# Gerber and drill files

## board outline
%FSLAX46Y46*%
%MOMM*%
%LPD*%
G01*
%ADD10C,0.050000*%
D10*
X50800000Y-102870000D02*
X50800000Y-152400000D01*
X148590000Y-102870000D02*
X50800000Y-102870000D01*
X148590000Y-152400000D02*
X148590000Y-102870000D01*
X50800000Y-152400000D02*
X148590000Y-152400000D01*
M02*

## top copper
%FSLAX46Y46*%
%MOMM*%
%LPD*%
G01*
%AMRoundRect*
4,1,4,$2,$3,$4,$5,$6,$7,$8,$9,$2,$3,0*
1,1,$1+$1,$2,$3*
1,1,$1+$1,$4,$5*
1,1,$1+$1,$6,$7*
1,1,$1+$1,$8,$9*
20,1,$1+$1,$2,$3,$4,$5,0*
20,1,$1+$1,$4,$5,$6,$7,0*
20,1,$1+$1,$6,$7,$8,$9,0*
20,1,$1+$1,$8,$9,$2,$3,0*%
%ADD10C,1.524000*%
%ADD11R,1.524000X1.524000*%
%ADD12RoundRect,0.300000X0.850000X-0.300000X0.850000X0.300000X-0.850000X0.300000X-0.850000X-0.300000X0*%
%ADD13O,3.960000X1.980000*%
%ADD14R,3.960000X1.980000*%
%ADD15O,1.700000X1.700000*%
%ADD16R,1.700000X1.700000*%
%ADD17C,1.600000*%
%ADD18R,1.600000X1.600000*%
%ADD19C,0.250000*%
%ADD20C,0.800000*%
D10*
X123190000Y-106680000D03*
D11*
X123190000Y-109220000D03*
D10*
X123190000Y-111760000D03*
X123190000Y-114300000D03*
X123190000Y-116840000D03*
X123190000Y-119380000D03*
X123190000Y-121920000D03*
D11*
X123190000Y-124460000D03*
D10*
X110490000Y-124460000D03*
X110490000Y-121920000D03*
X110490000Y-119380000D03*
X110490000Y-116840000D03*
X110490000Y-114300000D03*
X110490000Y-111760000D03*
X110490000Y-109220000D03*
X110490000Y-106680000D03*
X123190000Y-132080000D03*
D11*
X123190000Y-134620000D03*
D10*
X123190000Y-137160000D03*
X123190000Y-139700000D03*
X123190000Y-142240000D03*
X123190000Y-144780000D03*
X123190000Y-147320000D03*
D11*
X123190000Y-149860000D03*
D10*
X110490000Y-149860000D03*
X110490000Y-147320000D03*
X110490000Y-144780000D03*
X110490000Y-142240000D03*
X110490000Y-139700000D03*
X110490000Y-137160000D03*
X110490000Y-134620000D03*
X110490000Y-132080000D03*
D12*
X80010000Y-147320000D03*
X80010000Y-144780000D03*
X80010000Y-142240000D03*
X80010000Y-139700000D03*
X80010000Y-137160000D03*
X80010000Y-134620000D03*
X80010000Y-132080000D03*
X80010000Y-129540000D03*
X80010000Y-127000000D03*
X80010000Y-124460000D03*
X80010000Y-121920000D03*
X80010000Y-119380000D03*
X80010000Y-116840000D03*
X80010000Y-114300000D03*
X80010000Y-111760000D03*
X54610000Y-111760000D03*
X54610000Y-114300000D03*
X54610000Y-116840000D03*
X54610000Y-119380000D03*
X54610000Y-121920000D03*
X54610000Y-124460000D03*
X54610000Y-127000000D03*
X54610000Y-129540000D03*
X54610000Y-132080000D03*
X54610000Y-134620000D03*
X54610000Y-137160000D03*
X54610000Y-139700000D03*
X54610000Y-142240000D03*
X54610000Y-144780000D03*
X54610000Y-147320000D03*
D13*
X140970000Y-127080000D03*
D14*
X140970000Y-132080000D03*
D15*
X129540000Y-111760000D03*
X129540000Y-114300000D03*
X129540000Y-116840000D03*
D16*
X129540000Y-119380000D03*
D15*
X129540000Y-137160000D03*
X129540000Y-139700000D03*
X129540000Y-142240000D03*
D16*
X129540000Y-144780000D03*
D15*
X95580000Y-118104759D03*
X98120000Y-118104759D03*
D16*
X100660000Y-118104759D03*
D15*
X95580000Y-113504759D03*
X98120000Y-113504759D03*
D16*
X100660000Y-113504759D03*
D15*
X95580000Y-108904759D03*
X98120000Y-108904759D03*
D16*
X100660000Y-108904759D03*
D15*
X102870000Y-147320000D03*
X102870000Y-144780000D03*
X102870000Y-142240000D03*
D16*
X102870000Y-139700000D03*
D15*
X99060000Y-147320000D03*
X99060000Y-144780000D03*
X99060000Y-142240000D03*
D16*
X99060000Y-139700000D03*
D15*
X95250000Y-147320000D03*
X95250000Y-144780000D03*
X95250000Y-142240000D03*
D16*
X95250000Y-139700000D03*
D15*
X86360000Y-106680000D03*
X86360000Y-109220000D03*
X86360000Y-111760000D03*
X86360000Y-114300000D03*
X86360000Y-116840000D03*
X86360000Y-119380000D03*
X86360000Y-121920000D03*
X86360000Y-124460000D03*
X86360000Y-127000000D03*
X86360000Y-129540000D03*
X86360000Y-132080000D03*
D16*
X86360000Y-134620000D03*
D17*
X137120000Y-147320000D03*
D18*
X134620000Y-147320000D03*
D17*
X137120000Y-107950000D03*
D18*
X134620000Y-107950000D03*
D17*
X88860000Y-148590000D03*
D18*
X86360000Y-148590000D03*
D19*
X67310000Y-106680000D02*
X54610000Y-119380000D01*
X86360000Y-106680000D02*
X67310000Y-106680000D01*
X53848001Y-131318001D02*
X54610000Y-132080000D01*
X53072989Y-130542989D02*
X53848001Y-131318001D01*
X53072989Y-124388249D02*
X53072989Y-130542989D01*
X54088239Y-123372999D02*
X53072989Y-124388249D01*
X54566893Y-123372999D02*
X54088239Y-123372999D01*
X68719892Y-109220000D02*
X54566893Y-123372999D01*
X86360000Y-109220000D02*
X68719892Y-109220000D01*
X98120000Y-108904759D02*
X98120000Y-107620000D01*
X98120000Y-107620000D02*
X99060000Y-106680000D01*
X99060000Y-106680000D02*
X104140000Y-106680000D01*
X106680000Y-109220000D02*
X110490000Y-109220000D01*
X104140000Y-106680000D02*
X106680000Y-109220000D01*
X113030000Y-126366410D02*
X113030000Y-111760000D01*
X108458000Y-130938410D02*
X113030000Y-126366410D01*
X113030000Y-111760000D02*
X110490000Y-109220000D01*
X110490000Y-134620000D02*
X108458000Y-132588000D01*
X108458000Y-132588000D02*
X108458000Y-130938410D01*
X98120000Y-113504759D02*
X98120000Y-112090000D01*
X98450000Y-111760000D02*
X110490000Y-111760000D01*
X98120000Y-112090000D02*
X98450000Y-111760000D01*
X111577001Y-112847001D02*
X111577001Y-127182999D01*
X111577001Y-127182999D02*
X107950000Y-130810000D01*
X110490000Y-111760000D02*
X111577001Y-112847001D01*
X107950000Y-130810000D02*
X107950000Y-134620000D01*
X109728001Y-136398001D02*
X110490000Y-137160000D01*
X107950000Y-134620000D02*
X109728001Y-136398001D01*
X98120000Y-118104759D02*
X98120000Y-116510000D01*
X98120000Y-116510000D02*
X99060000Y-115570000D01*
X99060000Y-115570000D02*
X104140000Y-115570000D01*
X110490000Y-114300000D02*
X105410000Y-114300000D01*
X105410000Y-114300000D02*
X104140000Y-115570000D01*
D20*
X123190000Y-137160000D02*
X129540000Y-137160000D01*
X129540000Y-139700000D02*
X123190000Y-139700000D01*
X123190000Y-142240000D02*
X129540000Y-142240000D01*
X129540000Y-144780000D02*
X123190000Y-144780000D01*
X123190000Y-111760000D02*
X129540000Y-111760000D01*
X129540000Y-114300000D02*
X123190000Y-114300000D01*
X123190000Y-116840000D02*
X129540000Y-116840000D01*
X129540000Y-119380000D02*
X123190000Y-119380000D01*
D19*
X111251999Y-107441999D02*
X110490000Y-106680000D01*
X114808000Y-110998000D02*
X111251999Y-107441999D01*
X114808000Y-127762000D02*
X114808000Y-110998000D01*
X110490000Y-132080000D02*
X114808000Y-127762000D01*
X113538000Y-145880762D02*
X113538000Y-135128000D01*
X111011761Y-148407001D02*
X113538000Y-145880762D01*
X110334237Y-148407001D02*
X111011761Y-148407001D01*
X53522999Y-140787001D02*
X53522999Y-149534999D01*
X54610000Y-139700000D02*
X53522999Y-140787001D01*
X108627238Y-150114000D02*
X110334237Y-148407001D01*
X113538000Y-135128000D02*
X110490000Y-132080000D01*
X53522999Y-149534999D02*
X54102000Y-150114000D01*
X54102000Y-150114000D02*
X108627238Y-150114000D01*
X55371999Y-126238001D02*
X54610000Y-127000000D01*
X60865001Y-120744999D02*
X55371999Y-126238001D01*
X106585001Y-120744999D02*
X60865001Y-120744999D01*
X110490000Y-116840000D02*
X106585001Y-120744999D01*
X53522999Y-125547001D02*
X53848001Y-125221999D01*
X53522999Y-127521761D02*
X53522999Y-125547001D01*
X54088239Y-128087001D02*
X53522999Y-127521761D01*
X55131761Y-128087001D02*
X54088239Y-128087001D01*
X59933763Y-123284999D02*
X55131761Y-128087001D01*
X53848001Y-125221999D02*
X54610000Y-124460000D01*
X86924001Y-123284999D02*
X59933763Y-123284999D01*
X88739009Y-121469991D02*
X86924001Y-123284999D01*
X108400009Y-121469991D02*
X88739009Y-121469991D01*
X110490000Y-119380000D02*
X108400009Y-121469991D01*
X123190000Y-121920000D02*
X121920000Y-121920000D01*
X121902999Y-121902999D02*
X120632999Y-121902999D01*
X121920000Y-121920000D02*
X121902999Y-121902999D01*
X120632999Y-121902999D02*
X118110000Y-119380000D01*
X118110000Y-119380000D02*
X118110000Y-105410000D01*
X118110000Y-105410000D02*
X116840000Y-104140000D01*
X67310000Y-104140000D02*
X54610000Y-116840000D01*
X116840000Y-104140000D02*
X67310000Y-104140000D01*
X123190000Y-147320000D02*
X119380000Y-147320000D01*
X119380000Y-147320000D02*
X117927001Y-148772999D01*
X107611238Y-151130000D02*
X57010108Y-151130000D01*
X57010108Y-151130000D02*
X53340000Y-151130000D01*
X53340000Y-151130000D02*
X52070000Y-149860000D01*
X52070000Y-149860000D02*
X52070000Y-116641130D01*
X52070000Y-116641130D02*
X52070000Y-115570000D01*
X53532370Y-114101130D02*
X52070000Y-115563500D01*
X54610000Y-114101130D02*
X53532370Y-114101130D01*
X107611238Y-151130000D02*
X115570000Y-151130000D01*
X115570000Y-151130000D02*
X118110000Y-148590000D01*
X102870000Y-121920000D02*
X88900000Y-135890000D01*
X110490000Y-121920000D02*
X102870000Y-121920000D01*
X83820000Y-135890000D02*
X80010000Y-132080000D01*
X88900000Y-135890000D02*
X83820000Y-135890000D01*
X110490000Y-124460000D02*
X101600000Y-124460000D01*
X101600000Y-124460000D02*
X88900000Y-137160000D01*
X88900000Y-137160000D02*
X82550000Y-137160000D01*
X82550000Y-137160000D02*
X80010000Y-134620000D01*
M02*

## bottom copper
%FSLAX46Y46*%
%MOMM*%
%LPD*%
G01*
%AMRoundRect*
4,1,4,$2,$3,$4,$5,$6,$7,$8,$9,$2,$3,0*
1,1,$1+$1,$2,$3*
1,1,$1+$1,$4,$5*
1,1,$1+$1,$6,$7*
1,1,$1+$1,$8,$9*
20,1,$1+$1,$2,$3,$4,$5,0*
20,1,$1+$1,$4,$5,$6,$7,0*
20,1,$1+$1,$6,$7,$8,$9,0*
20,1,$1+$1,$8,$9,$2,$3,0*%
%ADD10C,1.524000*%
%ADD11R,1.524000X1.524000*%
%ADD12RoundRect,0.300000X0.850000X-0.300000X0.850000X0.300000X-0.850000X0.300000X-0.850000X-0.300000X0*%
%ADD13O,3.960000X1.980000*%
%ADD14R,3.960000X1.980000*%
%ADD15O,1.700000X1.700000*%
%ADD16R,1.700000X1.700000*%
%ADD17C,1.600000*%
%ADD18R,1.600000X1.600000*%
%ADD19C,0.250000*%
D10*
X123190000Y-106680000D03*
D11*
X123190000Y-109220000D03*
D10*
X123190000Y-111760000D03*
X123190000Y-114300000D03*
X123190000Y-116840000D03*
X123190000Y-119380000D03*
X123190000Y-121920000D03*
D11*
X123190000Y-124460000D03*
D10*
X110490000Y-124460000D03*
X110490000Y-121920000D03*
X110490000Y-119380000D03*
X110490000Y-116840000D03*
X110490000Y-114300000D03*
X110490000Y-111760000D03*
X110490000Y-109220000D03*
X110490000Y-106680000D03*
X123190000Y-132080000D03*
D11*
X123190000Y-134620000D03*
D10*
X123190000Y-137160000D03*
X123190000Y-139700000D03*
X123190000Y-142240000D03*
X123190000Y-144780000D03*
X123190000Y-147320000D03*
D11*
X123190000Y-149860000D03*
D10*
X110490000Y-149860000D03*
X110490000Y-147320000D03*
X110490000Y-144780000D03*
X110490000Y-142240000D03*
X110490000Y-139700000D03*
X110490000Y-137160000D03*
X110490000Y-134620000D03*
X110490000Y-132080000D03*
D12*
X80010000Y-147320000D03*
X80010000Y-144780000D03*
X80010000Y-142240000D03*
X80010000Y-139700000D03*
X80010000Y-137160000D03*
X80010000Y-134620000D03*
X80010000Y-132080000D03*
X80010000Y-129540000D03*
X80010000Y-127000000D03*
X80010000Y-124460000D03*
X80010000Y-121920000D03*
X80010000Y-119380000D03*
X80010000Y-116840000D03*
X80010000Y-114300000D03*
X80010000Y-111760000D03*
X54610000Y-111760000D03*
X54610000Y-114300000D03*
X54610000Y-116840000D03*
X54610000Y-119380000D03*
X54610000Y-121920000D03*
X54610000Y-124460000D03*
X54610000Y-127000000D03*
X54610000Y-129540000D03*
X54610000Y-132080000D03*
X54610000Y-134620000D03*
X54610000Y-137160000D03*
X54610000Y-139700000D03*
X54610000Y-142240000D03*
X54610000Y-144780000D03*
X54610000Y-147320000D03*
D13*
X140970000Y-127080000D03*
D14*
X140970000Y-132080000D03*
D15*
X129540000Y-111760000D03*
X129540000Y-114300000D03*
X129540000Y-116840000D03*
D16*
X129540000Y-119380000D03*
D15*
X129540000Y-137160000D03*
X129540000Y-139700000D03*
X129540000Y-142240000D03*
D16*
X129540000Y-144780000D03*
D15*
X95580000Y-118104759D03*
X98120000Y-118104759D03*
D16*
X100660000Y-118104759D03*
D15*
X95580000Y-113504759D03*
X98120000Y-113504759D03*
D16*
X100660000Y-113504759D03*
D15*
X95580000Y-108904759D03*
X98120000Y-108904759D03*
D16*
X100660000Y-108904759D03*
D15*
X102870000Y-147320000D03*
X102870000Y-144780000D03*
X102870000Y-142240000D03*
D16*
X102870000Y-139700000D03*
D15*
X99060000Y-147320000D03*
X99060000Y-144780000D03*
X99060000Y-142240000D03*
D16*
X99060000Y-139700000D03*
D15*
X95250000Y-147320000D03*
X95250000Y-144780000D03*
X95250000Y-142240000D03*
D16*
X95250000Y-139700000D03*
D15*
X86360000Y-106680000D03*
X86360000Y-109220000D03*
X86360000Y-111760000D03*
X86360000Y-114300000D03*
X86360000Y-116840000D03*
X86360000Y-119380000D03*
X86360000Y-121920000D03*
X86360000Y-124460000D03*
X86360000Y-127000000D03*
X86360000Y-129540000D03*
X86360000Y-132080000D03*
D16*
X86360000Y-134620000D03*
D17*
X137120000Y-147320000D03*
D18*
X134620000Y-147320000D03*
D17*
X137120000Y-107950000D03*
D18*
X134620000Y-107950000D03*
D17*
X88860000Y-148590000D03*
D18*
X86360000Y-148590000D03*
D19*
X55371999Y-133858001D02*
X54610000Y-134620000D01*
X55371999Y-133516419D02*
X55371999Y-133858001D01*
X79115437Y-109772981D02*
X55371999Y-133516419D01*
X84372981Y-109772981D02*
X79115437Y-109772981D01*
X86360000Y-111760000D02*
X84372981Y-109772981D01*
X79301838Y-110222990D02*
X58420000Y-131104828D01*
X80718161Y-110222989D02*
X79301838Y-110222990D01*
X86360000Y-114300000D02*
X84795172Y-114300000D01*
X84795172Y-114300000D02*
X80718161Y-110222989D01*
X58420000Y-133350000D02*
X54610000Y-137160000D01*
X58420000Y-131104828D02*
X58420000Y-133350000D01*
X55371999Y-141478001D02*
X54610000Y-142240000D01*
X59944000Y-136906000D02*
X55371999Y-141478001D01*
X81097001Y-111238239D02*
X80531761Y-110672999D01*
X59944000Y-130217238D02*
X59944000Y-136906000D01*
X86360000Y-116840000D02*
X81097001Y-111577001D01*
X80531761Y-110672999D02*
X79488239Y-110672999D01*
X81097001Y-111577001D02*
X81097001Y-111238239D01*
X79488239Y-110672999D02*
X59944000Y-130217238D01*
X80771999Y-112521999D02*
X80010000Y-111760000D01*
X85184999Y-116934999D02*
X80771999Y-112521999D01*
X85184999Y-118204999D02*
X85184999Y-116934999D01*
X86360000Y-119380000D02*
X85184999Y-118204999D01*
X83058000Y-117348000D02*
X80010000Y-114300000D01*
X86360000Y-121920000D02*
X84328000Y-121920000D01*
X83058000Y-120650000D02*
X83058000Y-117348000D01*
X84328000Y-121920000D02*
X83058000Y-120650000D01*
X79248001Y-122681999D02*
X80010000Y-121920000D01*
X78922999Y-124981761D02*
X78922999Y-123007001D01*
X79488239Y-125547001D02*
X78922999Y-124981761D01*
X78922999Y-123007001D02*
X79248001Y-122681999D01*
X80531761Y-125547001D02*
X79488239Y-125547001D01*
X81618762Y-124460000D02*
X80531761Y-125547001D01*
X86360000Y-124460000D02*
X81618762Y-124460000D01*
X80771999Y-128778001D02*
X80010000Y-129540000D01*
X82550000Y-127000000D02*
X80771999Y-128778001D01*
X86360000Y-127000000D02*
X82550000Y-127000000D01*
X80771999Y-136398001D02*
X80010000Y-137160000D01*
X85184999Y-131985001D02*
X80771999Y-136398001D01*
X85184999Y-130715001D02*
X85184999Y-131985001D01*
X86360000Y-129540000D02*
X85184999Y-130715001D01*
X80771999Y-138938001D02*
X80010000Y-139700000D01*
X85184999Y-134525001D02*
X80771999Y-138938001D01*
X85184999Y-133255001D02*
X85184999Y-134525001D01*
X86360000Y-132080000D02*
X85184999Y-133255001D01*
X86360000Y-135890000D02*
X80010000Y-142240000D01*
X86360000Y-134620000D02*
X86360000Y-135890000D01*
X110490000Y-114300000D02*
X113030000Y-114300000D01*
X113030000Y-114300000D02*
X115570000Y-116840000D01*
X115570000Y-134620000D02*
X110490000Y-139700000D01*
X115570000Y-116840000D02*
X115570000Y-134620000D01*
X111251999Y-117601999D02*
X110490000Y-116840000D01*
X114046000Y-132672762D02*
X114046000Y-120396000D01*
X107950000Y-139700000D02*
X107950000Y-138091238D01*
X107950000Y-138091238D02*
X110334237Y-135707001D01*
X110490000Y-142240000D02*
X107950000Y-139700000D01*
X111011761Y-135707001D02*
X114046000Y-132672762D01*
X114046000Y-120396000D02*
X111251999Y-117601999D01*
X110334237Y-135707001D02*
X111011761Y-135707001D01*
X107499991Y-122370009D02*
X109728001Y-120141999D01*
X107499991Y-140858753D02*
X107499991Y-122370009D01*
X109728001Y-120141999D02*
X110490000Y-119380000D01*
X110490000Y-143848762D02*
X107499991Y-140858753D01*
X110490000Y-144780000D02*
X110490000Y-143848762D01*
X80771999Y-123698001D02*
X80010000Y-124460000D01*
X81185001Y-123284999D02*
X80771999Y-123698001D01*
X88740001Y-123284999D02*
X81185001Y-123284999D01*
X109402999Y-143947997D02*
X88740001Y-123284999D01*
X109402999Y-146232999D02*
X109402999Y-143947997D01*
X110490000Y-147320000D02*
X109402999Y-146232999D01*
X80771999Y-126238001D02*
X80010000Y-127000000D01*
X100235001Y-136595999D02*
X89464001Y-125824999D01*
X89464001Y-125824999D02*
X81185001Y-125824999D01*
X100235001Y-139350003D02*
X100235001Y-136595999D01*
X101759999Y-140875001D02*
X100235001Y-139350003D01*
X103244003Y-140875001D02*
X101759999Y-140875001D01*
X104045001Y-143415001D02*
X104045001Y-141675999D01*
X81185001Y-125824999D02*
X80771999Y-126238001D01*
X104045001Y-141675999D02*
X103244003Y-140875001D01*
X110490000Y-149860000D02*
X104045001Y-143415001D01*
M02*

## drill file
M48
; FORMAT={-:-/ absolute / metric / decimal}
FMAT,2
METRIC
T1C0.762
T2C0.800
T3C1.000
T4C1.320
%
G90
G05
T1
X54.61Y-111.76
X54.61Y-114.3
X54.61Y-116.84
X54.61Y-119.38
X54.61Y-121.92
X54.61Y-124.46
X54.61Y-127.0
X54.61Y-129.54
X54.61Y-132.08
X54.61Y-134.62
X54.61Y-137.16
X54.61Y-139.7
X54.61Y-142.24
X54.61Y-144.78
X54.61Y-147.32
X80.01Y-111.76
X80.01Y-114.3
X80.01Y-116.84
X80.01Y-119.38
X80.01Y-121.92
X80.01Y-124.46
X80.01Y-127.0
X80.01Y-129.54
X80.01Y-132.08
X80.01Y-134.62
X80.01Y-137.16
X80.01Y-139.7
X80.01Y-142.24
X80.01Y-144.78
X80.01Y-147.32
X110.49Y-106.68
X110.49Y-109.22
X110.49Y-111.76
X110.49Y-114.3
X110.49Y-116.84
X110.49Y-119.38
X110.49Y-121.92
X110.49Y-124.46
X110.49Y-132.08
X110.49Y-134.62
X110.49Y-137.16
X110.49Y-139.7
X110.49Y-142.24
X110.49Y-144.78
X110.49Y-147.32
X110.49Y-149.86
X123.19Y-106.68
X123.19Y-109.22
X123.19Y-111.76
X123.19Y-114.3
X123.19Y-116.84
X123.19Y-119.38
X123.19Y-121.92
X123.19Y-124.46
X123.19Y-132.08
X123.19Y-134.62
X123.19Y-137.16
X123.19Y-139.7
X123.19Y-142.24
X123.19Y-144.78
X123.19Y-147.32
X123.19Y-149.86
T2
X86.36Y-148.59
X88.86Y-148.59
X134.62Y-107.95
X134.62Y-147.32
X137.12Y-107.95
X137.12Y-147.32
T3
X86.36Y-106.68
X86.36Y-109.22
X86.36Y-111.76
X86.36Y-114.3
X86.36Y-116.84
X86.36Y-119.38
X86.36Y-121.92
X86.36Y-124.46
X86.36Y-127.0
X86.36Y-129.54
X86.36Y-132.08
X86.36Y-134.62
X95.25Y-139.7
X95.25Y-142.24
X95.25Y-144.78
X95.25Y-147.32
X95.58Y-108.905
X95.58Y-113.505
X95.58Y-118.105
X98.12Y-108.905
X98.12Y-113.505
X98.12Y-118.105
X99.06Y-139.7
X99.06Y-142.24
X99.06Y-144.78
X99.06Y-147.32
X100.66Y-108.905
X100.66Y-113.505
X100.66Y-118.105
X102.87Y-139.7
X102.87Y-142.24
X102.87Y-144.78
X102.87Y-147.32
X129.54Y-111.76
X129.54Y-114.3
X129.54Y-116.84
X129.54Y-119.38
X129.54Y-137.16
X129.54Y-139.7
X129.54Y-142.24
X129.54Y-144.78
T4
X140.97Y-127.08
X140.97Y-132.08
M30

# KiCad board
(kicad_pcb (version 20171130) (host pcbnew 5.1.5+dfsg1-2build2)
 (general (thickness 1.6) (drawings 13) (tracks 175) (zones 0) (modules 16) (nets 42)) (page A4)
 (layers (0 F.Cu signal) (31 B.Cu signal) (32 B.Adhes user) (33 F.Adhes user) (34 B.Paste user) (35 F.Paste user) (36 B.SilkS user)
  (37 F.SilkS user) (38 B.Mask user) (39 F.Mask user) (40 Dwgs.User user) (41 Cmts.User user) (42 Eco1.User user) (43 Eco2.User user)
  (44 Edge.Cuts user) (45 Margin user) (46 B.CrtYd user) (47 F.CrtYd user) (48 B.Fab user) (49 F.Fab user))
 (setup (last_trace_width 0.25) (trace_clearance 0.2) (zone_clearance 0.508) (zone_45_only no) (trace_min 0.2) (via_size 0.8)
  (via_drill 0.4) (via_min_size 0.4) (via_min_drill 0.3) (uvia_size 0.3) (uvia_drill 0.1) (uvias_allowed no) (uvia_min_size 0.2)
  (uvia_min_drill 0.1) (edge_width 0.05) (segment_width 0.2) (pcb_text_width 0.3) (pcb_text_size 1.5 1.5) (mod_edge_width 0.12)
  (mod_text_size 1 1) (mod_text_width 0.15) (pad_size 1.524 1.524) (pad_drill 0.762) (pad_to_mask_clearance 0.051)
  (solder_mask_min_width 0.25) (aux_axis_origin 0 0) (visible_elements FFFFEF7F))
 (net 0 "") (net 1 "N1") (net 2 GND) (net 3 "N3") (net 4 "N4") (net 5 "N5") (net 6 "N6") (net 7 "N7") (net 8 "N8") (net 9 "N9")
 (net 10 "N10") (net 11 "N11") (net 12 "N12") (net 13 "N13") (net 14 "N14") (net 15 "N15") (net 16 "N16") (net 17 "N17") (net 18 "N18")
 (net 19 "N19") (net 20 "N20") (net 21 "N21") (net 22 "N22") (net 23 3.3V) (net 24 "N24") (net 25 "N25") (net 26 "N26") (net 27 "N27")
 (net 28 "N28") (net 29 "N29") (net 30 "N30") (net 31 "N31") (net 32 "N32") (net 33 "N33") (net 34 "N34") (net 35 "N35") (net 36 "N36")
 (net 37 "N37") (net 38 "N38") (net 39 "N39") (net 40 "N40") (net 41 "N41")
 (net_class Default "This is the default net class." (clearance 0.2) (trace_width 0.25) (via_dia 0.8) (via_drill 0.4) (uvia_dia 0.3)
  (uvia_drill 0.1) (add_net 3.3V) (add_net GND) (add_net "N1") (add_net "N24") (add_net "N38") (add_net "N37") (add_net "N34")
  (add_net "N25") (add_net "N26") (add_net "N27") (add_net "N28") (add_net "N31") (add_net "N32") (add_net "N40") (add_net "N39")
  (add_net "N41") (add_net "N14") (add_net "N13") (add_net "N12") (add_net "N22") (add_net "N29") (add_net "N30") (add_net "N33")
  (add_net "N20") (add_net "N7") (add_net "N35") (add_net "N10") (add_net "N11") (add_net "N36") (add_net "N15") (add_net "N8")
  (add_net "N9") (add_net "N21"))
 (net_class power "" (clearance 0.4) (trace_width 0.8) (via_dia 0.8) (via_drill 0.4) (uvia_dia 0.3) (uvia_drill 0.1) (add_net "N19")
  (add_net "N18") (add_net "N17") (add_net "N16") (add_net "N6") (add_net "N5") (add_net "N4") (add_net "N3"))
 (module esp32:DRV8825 (layer F.Cu) (at 116.84 115.57)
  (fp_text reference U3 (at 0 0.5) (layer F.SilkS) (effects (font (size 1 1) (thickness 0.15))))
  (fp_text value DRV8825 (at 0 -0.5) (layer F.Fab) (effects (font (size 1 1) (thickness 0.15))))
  (pad 16 thru_hole circle (at 6.35 -8.89) (size 1.524 1.524) (drill 0.762) (layers *.Cu *.Mask) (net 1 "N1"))
  (pad 15 thru_hole rect (at 6.35 -6.35) (size 1.524 1.524) (drill 0.762) (layers *.Cu *.Mask) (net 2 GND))
  (pad 14 thru_hole circle (at 6.35 -3.81) (size 1.524 1.524) (drill 0.762) (layers *.Cu *.Mask) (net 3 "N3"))
  (pad 13 thru_hole circle (at 6.35 -1.27) (size 1.524 1.524) (drill 0.762) (layers *.Cu *.Mask) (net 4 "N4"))
  (pad 12 thru_hole circle (at 6.35 1.27) (size 1.524 1.524) (drill 0.762) (layers *.Cu *.Mask) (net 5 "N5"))
  (pad 11 thru_hole circle (at 6.35 3.81) (size 1.524 1.524) (drill 0.762) (layers *.Cu *.Mask) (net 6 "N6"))
  (pad 10 thru_hole circle (at 6.35 6.35) (size 1.524 1.524) (drill 0.762) (layers *.Cu *.Mask) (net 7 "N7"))
  (pad 9 thru_hole rect (at 6.35 8.89) (size 1.524 1.524) (drill 0.762) (layers *.Cu *.Mask) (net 2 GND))
  (pad 8 thru_hole circle (at -6.35 8.89) (size 1.524 1.524) (drill 0.762) (layers *.Cu *.Mask) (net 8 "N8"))
  (pad 7 thru_hole circle (at -6.35 6.35) (size 1.524 1.524) (drill 0.762) (layers *.Cu *.Mask) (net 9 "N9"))
  (pad 6 thru_hole circle (at -6.35 3.81) (size 1.524 1.524) (drill 0.762) (layers *.Cu *.Mask) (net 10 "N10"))
  (pad 5 thru_hole circle (at -6.35 1.27) (size 1.524 1.524) (drill 0.762) (layers *.Cu *.Mask) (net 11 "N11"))
  (pad 4 thru_hole circle (at -6.35 -1.27) (size 1.524 1.524) (drill 0.762) (layers *.Cu *.Mask) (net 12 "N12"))
  (pad 3 thru_hole circle (at -6.35 -3.81) (size 1.524 1.524) (drill 0.762) (layers *.Cu *.Mask) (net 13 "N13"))
  (pad 2 thru_hole circle (at -6.35 -6.35) (size 1.524 1.524) (drill 0.762) (layers *.Cu *.Mask) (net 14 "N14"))
  (pad 1 thru_hole circle (at -6.35 -8.89) (size 1.524 1.524) (drill 0.762) (layers *.Cu *.Mask) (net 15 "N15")))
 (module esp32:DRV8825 (layer F.Cu) (at 116.84 140.97)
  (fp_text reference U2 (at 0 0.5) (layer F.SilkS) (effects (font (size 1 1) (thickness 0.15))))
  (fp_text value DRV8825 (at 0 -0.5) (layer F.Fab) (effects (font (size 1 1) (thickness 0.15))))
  (pad 16 thru_hole circle (at 6.35 -8.89) (size 1.524 1.524) (drill 0.762) (layers *.Cu *.Mask) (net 1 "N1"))
  (pad 15 thru_hole rect (at 6.35 -6.35) (size 1.524 1.524) (drill 0.762) (layers *.Cu *.Mask) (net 2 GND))
  (pad 14 thru_hole circle (at 6.35 -3.81) (size 1.524 1.524) (drill 0.762) (layers *.Cu *.Mask) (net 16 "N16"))
  (pad 13 thru_hole circle (at 6.35 -1.27) (size 1.524 1.524) (drill 0.762) (layers *.Cu *.Mask) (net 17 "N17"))
  (pad 12 thru_hole circle (at 6.35 1.27) (size 1.524 1.524) (drill 0.762) (layers *.Cu *.Mask) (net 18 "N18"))
  (pad 11 thru_hole circle (at 6.35 3.81) (size 1.524 1.524) (drill 0.762) (layers *.Cu *.Mask) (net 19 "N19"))
  (pad 10 thru_hole circle (at 6.35 6.35) (size 1.524 1.524) (drill 0.762) (layers *.Cu *.Mask) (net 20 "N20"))
  (pad 9 thru_hole rect (at 6.35 8.89) (size 1.524 1.524) (drill 0.762) (layers *.Cu *.Mask) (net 2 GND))
  (pad 8 thru_hole circle (at -6.35 8.89) (size 1.524 1.524) (drill 0.762) (layers *.Cu *.Mask) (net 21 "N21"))
  (pad 7 thru_hole circle (at -6.35 6.35) (size 1.524 1.524) (drill 0.762) (layers *.Cu *.Mask) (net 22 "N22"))
  (pad 6 thru_hole circle (at -6.35 3.81) (size 1.524 1.524) (drill 0.762) (layers *.Cu *.Mask) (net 10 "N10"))
  (pad 5 thru_hole circle (at -6.35 1.27) (size 1.524 1.524) (drill 0.762) (layers *.Cu *.Mask) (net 11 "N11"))
  (pad 4 thru_hole circle (at -6.35 -1.27) (size 1.524 1.524) (drill 0.762) (layers *.Cu *.Mask) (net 12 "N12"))
  (pad 3 thru_hole circle (at -6.35 -3.81) (size 1.524 1.524) (drill 0.762) (layers *.Cu *.Mask) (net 13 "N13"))
  (pad 2 thru_hole circle (at -6.35 -6.35) (size 1.524 1.524) (drill 0.762) (layers *.Cu *.Mask) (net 14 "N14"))
  (pad 1 thru_hole circle (at -6.35 -8.89) (size 1.524 1.524) (drill 0.762) (layers *.Cu *.Mask) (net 15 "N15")))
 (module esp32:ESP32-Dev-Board (layer F.Cu) (at 67.31 129.54 90)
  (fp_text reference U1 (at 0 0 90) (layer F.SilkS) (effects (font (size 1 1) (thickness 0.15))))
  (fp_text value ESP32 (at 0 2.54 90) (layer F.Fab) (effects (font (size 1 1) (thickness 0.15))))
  (pad 1 thru_hole roundrect (at -17.78 12.7 90) (size 1.2 2.3) (drill 0.762) (layers *.Cu *.Mask) (roundrect_rratio 0.25) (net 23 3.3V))
  (pad 2 thru_hole roundrect (at -15.24 12.7 90) (size 1.2 2.3) (drill 0.762) (layers *.Cu *.Mask) (roundrect_rratio 0.25) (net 2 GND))
  (pad 3 thru_hole roundrect (at -12.7 12.7 90) (size 1.2 2.3) (drill 0.762) (layers *.Cu *.Mask) (roundrect_rratio 0.25) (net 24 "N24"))
  (pad 4 thru_hole roundrect (at -10.16 12.7 90) (size 1.2 2.3) (drill 0.762) (layers *.Cu *.Mask) (roundrect_rratio 0.25) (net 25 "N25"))
  (pad 5 thru_hole roundrect (at -7.62 12.7 90) (size 1.2 2.3) (drill 0.762) (layers *.Cu *.Mask) (roundrect_rratio 0.25) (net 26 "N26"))
  (pad 6 thru_hole roundrect (at -5.08 12.7 90) (size 1.2 2.3) (drill 0.762) (layers *.Cu *.Mask) (roundrect_rratio 0.25) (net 8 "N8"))
  (pad 7 thru_hole roundrect (at -2.54 12.7 90) (size 1.2 2.3) (drill 0.762) (layers *.Cu *.Mask) (roundrect_rratio 0.25) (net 9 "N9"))
  (pad 8 thru_hole roundrect (at 0 12.7 90) (size 1.2 2.3) (drill 0.762) (layers *.Cu *.Mask) (roundrect_rratio 0.25) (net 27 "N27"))
  (pad 9 thru_hole roundrect (at 2.54 12.7 90) (size 1.2 2.3) (drill 0.762) (layers *.Cu *.Mask) (roundrect_rratio 0.25) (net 21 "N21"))
  (pad 10 thru_hole roundrect (at 5.08 12.7 90) (size 1.2 2.3) (drill 0.762) (layers *.Cu *.Mask) (roundrect_rratio 0.25) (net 22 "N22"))
  (pad 11 thru_hole roundrect (at 7.62 12.7 90) (size 1.2 2.3) (drill 0.762) (layers *.Cu *.Mask) (roundrect_rratio 0.25) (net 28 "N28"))
  (pad 12 thru_hole roundrect (at 10.16 12.7 90) (size 1.2 2.3) (drill 0.762) (layers *.Cu *.Mask) (roundrect_rratio 0.25) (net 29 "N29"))
  (pad 13 thru_hole roundrect (at 12.7 12.7 90) (size 1.2 2.3) (drill 0.762) (layers *.Cu *.Mask) (roundrect_rratio 0.25) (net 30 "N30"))
  (pad 14 thru_hole roundrect (at 15.24 12.7 90) (size 1.2 2.3) (drill 0.762) (layers *.Cu *.Mask) (roundrect_rratio 0.25) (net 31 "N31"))
  (pad 15 thru_hole roundrect (at 17.78 12.7 90) (size 1.2 2.3) (drill 0.762) (layers *.Cu *.Mask) (roundrect_rratio 0.25) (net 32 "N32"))
  (pad 16 thru_hole roundrect (at 17.78 -12.7 90) (size 1.2 2.3) (drill 0.762) (layers *.Cu *.Mask) (roundrect_rratio 0.25) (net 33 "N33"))
  (pad 17 thru_hole roundrect (at 15.24 -12.7 90) (size 1.2 2.3) (drill 0.762) (layers *.Cu *.Mask) (roundrect_rratio 0.25) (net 20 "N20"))
  (pad 18 thru_hole roundrect (at 12.7 -12.7 90) (size 1.2 2.3) (drill 0.762) (layers *.Cu *.Mask) (roundrect_rratio 0.25) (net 7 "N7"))
  (pad 19 thru_hole roundrect (at 10.16 -12.7 90) (size 1.2 2.3) (drill 0.762) (layers *.Cu *.Mask) (roundrect_rratio 0.25) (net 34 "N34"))
  (pad 20 thru_hole roundrect (at 7.62 -12.7 90) (size 1.2 2.3) (drill 0.762) (layers *.Cu *.Mask) (roundrect_rratio 0.25) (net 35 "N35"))
  (pad 21 thru_hole roundrect (at 5.08 -12.7 90) (size 1.2 2.3) (drill 0.762) (layers *.Cu *.Mask) (roundrect_rratio 0.25) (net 10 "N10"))
  (pad 22 thru_hole roundrect (at 2.54 -12.7 90) (size 1.2 2.3) (drill 0.762) (layers *.Cu *.Mask) (roundrect_rratio 0.25) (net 11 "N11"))
  (pad 23 thru_hole roundrect (at 0 -12.7 90) (size 1.2 2.3) (drill 0.762) (layers *.Cu *.Mask) (roundrect_rratio 0.25) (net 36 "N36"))
  (pad 24 thru_hole roundrect (at -2.54 -12.7 90) (size 1.2 2.3) (drill 0.762) (layers *.Cu *.Mask) (roundrect_rratio 0.25) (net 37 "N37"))
  (pad 25 thru_hole roundrect (at -5.08 -12.7 90) (size 1.2 2.3) (drill 0.762) (layers *.Cu *.Mask) (roundrect_rratio 0.25) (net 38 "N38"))
  (pad 26 thru_hole roundrect (at -7.62 -12.7 90) (size 1.2 2.3) (drill 0.762) (layers *.Cu *.Mask) (roundrect_rratio 0.25) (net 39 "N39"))
  (pad 27 thru_hole roundrect (at -10.16 -12.7 90) (size 1.2 2.3) (drill 0.762) (layers *.Cu *.Mask) (roundrect_rratio 0.25) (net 15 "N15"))
  (pad 28 thru_hole roundrect (at -12.7 -12.7 90) (size 1.2 2.3) (drill 0.762) (layers *.Cu *.Mask) (roundrect_rratio 0.25) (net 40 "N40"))
  (pad 29 thru_hole roundrect (at -15.24 -12.7 90) (size 1.2 2.3) (drill 0.762) (layers *.Cu *.Mask) (roundrect_rratio 0.25) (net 2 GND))
  (pad 30 thru_hole roundrect (at -17.78 -12.7 90) (size 1.2 2.3) (drill 0.762) (layers *.Cu *.Mask) (roundrect_rratio 0.25) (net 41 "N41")))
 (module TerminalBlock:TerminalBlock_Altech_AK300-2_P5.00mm (layer F.Cu) (at 140.97 132.08 90)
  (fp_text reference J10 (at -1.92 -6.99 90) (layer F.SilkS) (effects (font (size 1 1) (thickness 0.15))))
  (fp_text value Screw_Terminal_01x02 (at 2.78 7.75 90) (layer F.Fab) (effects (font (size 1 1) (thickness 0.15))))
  (pad 2 thru_hole oval (at 5 0 90) (size 1.98 3.96) (drill 1.32) (layers *.Cu *.Mask) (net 1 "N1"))
  (pad 1 thru_hole rect (at 0 0 90) (size 1.98 3.96) (drill 1.32) (layers *.Cu *.Mask) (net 2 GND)))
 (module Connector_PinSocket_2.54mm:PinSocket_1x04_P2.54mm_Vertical (layer F.Cu) (at 129.54 119.38 180)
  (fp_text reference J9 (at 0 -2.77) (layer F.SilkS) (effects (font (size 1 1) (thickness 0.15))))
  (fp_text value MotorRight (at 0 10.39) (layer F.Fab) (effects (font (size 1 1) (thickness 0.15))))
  (pad 4 thru_hole oval (at 0 7.62 180) (size 1.7 1.7) (drill 1) (layers *.Cu *.Mask) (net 3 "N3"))
  (pad 3 thru_hole oval (at 0 5.08 180) (size 1.7 1.7) (drill 1) (layers *.Cu *.Mask) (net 4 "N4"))
  (pad 2 thru_hole oval (at 0 2.54 180) (size 1.7 1.7) (drill 1) (layers *.Cu *.Mask) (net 5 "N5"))
  (pad 1 thru_hole rect (at 0 0 180) (size 1.7 1.7) (drill 1) (layers *.Cu *.Mask) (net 6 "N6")))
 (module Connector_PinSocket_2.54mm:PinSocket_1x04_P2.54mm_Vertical (layer F.Cu) (at 129.54 144.78 180)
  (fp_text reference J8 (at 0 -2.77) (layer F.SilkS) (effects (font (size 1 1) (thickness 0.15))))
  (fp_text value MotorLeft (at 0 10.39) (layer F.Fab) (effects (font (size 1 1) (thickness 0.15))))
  (pad 4 thru_hole oval (at 0 7.62 180) (size 1.7 1.7) (drill 1) (layers *.Cu *.Mask) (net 16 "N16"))
  (pad 3 thru_hole oval (at 0 5.08 180) (size 1.7 1.7) (drill 1) (layers *.Cu *.Mask) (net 17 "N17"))
  (pad 2 thru_hole oval (at 0 2.54 180) (size 1.7 1.7) (drill 1) (layers *.Cu *.Mask) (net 18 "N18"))
  (pad 1 thru_hole rect (at 0 0 180) (size 1.7 1.7) (drill 1) (layers *.Cu *.Mask) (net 19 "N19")))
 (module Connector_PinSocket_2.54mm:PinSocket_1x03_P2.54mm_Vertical (layer F.Cu) (at 100.66 118.104759 270)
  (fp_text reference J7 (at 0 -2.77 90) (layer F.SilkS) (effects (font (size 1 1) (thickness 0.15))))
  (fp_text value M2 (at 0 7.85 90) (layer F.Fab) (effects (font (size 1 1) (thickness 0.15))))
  (pad 3 thru_hole oval (at 0 5.08 270) (size 1.7 1.7) (drill 1) (layers *.Cu *.Mask) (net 23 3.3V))
  (pad 2 thru_hole oval (at 0 2.54 270) (size 1.7 1.7) (drill 1) (layers *.Cu *.Mask) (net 12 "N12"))
  (pad 1 thru_hole rect (at 0 0 270) (size 1.7 1.7) (drill 1) (layers *.Cu *.Mask) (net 2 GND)))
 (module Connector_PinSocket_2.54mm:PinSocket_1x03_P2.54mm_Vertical (layer F.Cu) (at 100.66 113.504759 270)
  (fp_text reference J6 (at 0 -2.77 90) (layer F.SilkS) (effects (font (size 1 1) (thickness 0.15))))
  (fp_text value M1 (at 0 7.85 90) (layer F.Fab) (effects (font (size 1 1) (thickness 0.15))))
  (pad 3 thru_hole oval (at 0 5.08 270) (size 1.7 1.7) (drill 1) (layers *.Cu *.Mask) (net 23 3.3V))
  (pad 2 thru_hole oval (at 0 2.54 270) (size 1.7 1.7) (drill 1) (layers *.Cu *.Mask) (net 13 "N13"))
  (pad 1 thru_hole rect (at 0 0 270) (size 1.7 1.7) (drill 1) (layers *.Cu *.Mask) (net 2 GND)))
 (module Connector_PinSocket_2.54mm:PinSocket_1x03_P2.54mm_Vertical (layer F.Cu) (at 100.66 108.904759 270)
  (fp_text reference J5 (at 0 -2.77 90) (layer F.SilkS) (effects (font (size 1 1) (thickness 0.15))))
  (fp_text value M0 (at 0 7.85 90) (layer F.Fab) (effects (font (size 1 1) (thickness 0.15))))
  (pad 3 thru_hole oval (at 0 5.08 270) (size 1.7 1.7) (drill 1) (layers *.Cu *.Mask) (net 23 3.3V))
  (pad 2 thru_hole oval (at 0 2.54 270) (size 1.7 1.7) (drill 1) (layers *.Cu *.Mask) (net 14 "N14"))
  (pad 1 thru_hole rect (at 0 0 270) (size 1.7 1.7) (drill 1) (layers *.Cu *.Mask) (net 2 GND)))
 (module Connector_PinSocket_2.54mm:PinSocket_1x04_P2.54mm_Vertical (layer F.Cu) (at 102.87 139.7)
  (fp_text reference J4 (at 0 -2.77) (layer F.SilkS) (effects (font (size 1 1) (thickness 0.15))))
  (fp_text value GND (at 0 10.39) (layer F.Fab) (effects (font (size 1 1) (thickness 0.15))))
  (pad 4 thru_hole oval (at 0 7.62) (size 1.7 1.7) (drill 1) (layers *.Cu *.Mask) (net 2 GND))
  (pad 3 thru_hole oval (at 0 5.08) (size 1.7 1.7) (drill 1) (layers *.Cu *.Mask) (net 2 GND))
  (pad 2 thru_hole oval (at 0 2.54) (size 1.7 1.7) (drill 1) (layers *.Cu *.Mask) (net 2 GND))
  (pad 1 thru_hole rect (at 0 0) (size 1.7 1.7) (drill 1) (layers *.Cu *.Mask) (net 2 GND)))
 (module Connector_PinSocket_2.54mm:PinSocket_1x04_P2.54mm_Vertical (layer F.Cu) (at 99.06 139.7)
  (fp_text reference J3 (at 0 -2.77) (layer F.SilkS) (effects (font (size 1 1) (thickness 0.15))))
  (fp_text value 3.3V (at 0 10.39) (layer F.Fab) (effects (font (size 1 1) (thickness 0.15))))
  (pad 4 thru_hole oval (at 0 7.62) (size 1.7 1.7) (drill 1) (layers *.Cu *.Mask) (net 23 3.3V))
  (pad 3 thru_hole oval (at 0 5.08) (size 1.7 1.7) (drill 1) (layers *.Cu *.Mask) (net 23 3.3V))
  (pad 2 thru_hole oval (at 0 2.54) (size 1.7 1.7) (drill 1) (layers *.Cu *.Mask) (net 23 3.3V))
  (pad 1 thru_hole rect (at 0 0) (size 1.7 1.7) (drill 1) (layers *.Cu *.Mask) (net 23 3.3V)))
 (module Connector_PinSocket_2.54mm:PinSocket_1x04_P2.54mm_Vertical (layer F.Cu) (at 95.25 139.7)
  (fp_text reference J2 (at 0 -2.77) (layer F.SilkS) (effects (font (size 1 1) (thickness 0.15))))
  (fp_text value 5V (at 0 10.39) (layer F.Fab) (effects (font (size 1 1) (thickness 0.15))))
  (pad 4 thru_hole oval (at 0 7.62) (size 1.7 1.7) (drill 1) (layers *.Cu *.Mask) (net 41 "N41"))
  (pad 3 thru_hole oval (at 0 5.08) (size 1.7 1.7) (drill 1) (layers *.Cu *.Mask) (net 41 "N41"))
  (pad 2 thru_hole oval (at 0 2.54) (size 1.7 1.7) (drill 1) (layers *.Cu *.Mask) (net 41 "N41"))
  (pad 1 thru_hole rect (at 0 0) (size 1.7 1.7) (drill 1) (layers *.Cu *.Mask) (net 41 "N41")))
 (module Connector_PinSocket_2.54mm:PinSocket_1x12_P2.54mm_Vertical (layer F.Cu) (at 86.36 134.62 180)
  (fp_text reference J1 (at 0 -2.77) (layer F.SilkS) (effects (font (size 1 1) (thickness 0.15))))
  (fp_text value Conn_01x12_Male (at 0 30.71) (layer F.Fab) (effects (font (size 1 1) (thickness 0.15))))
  (pad 12 thru_hole oval (at 0 27.94 180) (size 1.7 1.7) (drill 1) (layers *.Cu *.Mask) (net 34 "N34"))
  (pad 11 thru_hole oval (at 0 25.4 180) (size 1.7 1.7) (drill 1) (layers *.Cu *.Mask) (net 37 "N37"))
  (pad 10 thru_hole oval (at 0 22.86 180) (size 1.7 1.7) (drill 1) (layers *.Cu *.Mask) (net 38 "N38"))
  (pad 9 thru_hole oval (at 0 20.32 180) (size 1.7 1.7) (drill 1) (layers *.Cu *.Mask) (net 39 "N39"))
  (pad 8 thru_hole oval (at 0 17.78 180) (size 1.7 1.7) (drill 1) (layers *.Cu *.Mask) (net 40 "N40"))
  (pad 7 thru_hole oval (at 0 15.24 180) (size 1.7 1.7) (drill 1) (layers *.Cu *.Mask) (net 32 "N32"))
  (pad 6 thru_hole oval (at 0 12.7 180) (size 1.7 1.7) (drill 1) (layers *.Cu *.Mask) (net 31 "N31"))
  (pad 5 thru_hole oval (at 0 10.16 180) (size 1.7 1.7) (drill 1) (layers *.Cu *.Mask) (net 28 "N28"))
  (pad 4 thru_hole oval (at 0 7.62 180) (size 1.7 1.7) (drill 1) (layers *.Cu *.Mask) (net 27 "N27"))
  (pad 3 thru_hole oval (at 0 5.08 180) (size 1.7 1.7) (drill 1) (layers *.Cu *.Mask) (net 26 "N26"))
  (pad 2 thru_hole oval (at 0 2.54 180) (size 1.7 1.7) (drill 1) (layers *.Cu *.Mask) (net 25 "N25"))
  (pad 1 thru_hole rect (at 0 0 180) (size 1.7 1.7) (drill 1) (layers *.Cu *.Mask) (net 24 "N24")))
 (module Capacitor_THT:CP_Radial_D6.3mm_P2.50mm (layer F.Cu) (at 134.62 147.32)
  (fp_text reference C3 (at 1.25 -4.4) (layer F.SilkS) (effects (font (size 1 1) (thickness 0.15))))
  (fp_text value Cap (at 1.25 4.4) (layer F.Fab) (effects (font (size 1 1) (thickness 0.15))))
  (pad 2 thru_hole circle (at 2.5 0) (size 1.6 1.6) (drill 0.8) (layers *.Cu *.Mask) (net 2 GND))
  (pad 1 thru_hole rect (at 0 0) (size 1.6 1.6) (drill 0.8) (layers *.Cu *.Mask) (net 1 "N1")))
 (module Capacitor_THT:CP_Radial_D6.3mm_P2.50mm (layer F.Cu) (at 134.62 107.95)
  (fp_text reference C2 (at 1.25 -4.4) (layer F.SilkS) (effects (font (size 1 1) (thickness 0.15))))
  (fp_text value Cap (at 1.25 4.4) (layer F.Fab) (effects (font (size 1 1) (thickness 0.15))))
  (pad 2 thru_hole circle (at 2.5 0) (size 1.6 1.6) (drill 0.8) (layers *.Cu *.Mask) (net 2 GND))
  (pad 1 thru_hole rect (at 0 0) (size 1.6 1.6) (drill 0.8) (layers *.Cu *.Mask) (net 1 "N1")))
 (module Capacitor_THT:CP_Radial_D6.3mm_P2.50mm (layer F.Cu) (at 86.36 148.59)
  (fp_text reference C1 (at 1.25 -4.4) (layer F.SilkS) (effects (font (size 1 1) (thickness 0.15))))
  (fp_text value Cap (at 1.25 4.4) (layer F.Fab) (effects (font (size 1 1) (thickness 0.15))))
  (pad 2 thru_hole circle (at 2.5 0) (size 1.6 1.6) (drill 0.8) (layers *.Cu *.Mask) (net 2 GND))
  (pad 1 thru_hole rect (at 0 0) (size 1.6 1.6) (drill 0.8) (layers *.Cu *.Mask) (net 23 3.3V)))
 (gr_line (start 50.8 102.87) (end 50.8 152.4) (layer Edge.Cuts) (width 0.05))
 (gr_line (start 148.59 102.87) (end 50.8 102.87) (layer Edge.Cuts) (width 0.05))
 (gr_line (start 148.59 152.4) (end 148.59 102.87) (layer Edge.Cuts) (width 0.05))
 (gr_line (start 50.8 152.4) (end 148.59 152.4) (layer Edge.Cuts) (width 0.05))
 (segment (start 67.31 106.68) (end 54.61 119.38) (width 0.25) (layer F.Cu) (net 34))
 (segment (start 86.36 106.68) (end 67.31 106.68) (width 0.25) (layer F.Cu) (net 34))
 (segment (start 53.848001 131.318001) (end 54.61 132.08) (width 0.25) (layer F.Cu) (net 37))
 (segment (start 53.072989 130.542989) (end 53.848001 131.318001) (width 0.25) (layer F.Cu) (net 37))
 (segment (start 53.072989 124.388249) (end 53.072989 130.542989) (width 0.25) (layer F.Cu) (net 37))
 (segment (start 54.088239 123.372999) (end 53.072989 124.388249) (width 0.25) (layer F.Cu) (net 37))
 (segment (start 54.566893 123.372999) (end 54.088239 123.372999) (width 0.25) (layer F.Cu) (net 37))
 (segment (start 68.719892 109.22) (end 54.566893 123.372999) (width 0.25) (layer F.Cu) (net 37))
 (segment (start 86.36 109.22) (end 68.719892 109.22) (width 0.25) (layer F.Cu) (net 37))
 (segment (start 55.371999 133.858001) (end 54.61 134.62) (width 0.25) (layer B.Cu) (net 38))
 (segment (start 55.371999 133.516419) (end 55.371999 133.858001) (width 0.25) (layer B.Cu) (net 38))
 (segment (start 79.115437 109.772981) (end 55.371999 133.516419) (width 0.25) (layer B.Cu) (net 38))
 (segment (start 84.372981 109.772981) (end 79.115437 109.772981) (width 0.25) (layer B.Cu) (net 38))
 (segment (start 86.36 111.76) (end 84.372981 109.772981) (width 0.25) (layer B.Cu) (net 38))
 (segment (start 79.301838 110.22299) (end 58.42 131.104828) (width 0.25) (layer B.Cu) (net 39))
 (segment (start 80.718161 110.222989) (end 79.301838 110.22299) (width 0.25) (layer B.Cu) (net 39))
 (segment (start 86.36 114.3) (end 84.795172 114.3) (width 0.25) (layer B.Cu) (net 39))
 (segment (start 84.795172 114.3) (end 80.718161 110.222989) (width 0.25) (layer B.Cu) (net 39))
 (segment (start 58.42 133.35) (end 54.61 137.16) (width 0.25) (layer B.Cu) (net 39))
 (segment (start 58.42 131.104828) (end 58.42 133.35) (width 0.25) (layer B.Cu) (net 39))
 (segment (start 55.371999 141.478001) (end 54.61 142.24) (width 0.25) (layer B.Cu) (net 40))
 (segment (start 59.944 136.906) (end 55.371999 141.478001) (width 0.25) (layer B.Cu) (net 40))
 (segment (start 81.097001 111.238239) (end 80.531761 110.672999) (width 0.25) (layer B.Cu) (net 40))
 (segment (start 59.944 130.217238) (end 59.944 136.906) (width 0.25) (layer B.Cu) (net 40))
 (segment (start 86.36 116.84) (end 81.097001 111.577001) (width 0.25) (layer B.Cu) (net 40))
 (segment (start 80.531761 110.672999) (end 79.488239 110.672999) (width 0.25) (layer B.Cu) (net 40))
 (segment (start 81.097001 111.577001) (end 81.097001 111.238239) (width 0.25) (layer B.Cu) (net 40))
 (segment (start 79.488239 110.672999) (end 59.944 130.217238) (width 0.25) (layer B.Cu) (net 40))
 (segment (start 80.771999 112.521999) (end 80.01 111.76) (width 0.25) (layer B.Cu) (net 32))
 (segment (start 85.184999 116.934999) (end 80.771999 112.521999) (width 0.25) (layer B.Cu) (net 32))
 (segment (start 85.184999 118.204999) (end 85.184999 116.934999) (width 0.25) (layer B.Cu) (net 32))
 (segment (start 86.36 119.38) (end 85.184999 118.204999) (width 0.25) (layer B.Cu) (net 32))
 (segment (start 83.058 117.348) (end 80.01 114.3) (width 0.25) (layer B.Cu) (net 31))
 (segment (start 86.36 121.92) (end 84.328 121.92) (width 0.25) (layer B.Cu) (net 31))
 (segment (start 83.058 120.65) (end 83.058 117.348) (width 0.25) (layer B.Cu) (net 31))
 (segment (start 84.328 121.92) (end 83.058 120.65) (width 0.25) (layer B.Cu) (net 31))
 (segment (start 79.248001 122.681999) (end 80.01 121.92) (width 0.25) (layer B.Cu) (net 28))
 (segment (start 78.922999 124.981761) (end 78.922999 123.007001) (width 0.25) (layer B.Cu) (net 28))
 (segment (start 79.488239 125.547001) (end 78.922999 124.981761) (width 0.25) (layer B.Cu) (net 28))
 (segment (start 78.922999 123.007001) (end 79.248001 122.681999) (width 0.25) (layer B.Cu) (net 28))
 (segment (start 80.531761 125.547001) (end 79.488239 125.547001) (width 0.25) (layer B.Cu) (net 28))
 (segment (start 81.618762 124.46) (end 80.531761 125.547001) (width 0.25) (layer B.Cu) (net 28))
 (segment (start 86.36 124.46) (end 81.618762 124.46) (width 0.25) (layer B.Cu) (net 28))
 (segment (start 80.771999 128.778001) (end 80.01 129.54) (width 0.25) (layer B.Cu) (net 27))
 (segment (start 82.55 127) (end 80.771999 128.778001) (width 0.25) (layer B.Cu) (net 27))
 (segment (start 86.36 127) (end 82.55 127) (width 0.25) (layer B.Cu) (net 27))
 (segment (start 80.771999 136.398001) (end 80.01 137.16) (width 0.25) (layer B.Cu) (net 26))
 (segment (start 85.184999 131.985001) (end 80.771999 136.398001) (width 0.25) (layer B.Cu) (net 26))
 (segment (start 85.184999 130.715001) (end 85.184999 131.985001) (width 0.25) (layer B.Cu) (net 26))
 (segment (start 86.36 129.54) (end 85.184999 130.715001) (width 0.25) (layer B.Cu) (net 26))
 (segment (start 80.771999 138.938001) (end 80.01 139.7) (width 0.25) (layer B.Cu) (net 25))
 (segment (start 85.184999 134.525001) (end 80.771999 138.938001) (width 0.25) (layer B.Cu) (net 25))
 (segment (start 85.184999 133.255001) (end 85.184999 134.525001) (width 0.25) (layer B.Cu) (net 25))
 (segment (start 86.36 132.08) (end 85.184999 133.255001) (width 0.25) (layer B.Cu) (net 25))
 (segment (start 86.36 135.89) (end 80.01 142.24) (width 0.25) (layer B.Cu) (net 24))
 (segment (start 86.36 134.62) (end 86.36 135.89) (width 0.25) (layer B.Cu) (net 24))
 (segment (start 98.12 108.904759) (end 98.12 107.62) (width 0.25) (layer F.Cu) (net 14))
 (segment (start 98.12 107.62) (end 99.06 106.68) (width 0.25) (layer F.Cu) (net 14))
 (segment (start 99.06 106.68) (end 104.14 106.68) (width 0.25) (layer F.Cu) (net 14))
 (segment (start 106.68 109.22) (end 110.49 109.22) (width 0.25) (layer F.Cu) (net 14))
 (segment (start 104.14 106.68) (end 106.68 109.22) (width 0.25) (layer F.Cu) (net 14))
 (segment (start 113.03 126.36641) (end 113.03 111.76) (width 0.25) (layer F.Cu) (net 14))
 (segment (start 108.458 130.93841) (end 113.03 126.36641) (width 0.25) (layer F.Cu) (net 14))
 (segment (start 113.03 111.76) (end 110.49 109.22) (width 0.25) (layer F.Cu) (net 14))
 (segment (start 110.49 134.62) (end 108.458 132.588) (width 0.25) (layer F.Cu) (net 14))
 (segment (start 108.458 132.588) (end 108.458 130.93841) (width 0.25) (layer F.Cu) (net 14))
 (segment (start 98.12 113.504759) (end 98.12 112.09) (width 0.25) (layer F.Cu) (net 13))
 (segment (start 98.45 111.76) (end 110.49 111.76) (width 0.25) (layer F.Cu) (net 13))
 (segment (start 98.12 112.09) (end 98.45 111.76) (width 0.25) (layer F.Cu) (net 13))
 (segment (start 111.577001 112.847001) (end 111.577001 127.182999) (width 0.25) (layer F.Cu) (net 13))
 (segment (start 111.577001 127.182999) (end 107.95 130.81) (width 0.25) (layer F.Cu) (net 13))
 (segment (start 110.49 111.76) (end 111.577001 112.847001) (width 0.25) (layer F.Cu) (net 13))
 (segment (start 107.95 130.81) (end 107.95 134.62) (width 0.25) (layer F.Cu) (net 13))
 (segment (start 109.728001 136.398001) (end 110.49 137.16) (width 0.25) (layer F.Cu) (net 13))
 (segment (start 107.95 134.62) (end 109.728001 136.398001) (width 0.25) (layer F.Cu) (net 13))
 (segment (start 98.12 118.104759) (end 98.12 116.51) (width 0.25) (layer F.Cu) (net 12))
 (segment (start 98.12 116.51) (end 99.06 115.57) (width 0.25) (layer F.Cu) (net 12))
 (segment (start 99.06 115.57) (end 104.14 115.57) (width 0.25) (layer F.Cu) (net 12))
 (segment (start 110.49 114.3) (end 105.41 114.3) (width 0.25) (layer F.Cu) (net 12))
 (segment (start 105.41 114.3) (end 104.14 115.57) (width 0.25) (layer F.Cu) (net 12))
 (segment (start 110.49 114.3) (end 113.03 114.3) (width 0.25) (layer B.Cu) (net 12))
 (segment (start 113.03 114.3) (end 115.57 116.84) (width 0.25) (layer B.Cu) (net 12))
 (segment (start 115.57 134.62) (end 110.49 139.7) (width 0.25) (layer B.Cu) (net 12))
 (segment (start 115.57 116.84) (end 115.57 134.62) (width 0.25) (layer B.Cu) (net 12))
 (segment (start 123.19 137.16) (end 129.54 137.16) (width 0.8) (layer F.Cu) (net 16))
 (segment (start 129.54 139.7) (end 123.19 139.7) (width 0.8) (layer F.Cu) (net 17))
 (segment (start 123.19 142.24) (end 129.54 142.24) (width 0.8) (layer F.Cu) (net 18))
 (segment (start 129.54 144.78) (end 123.19 144.78) (width 0.8) (layer F.Cu) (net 19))
 (segment (start 123.19 111.76) (end 129.54 111.76) (width 0.8) (layer F.Cu) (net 3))
 (segment (start 129.54 114.3) (end 123.19 114.3) (width 0.8) (layer F.Cu) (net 4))
 (segment (start 123.19 116.84) (end 129.54 116.84) (width 0.8) (layer F.Cu) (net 5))
 (segment (start 129.54 119.38) (end 123.19 119.38) (width 0.8) (layer F.Cu) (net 6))
 (segment (start 111.251999 107.441999) (end 110.49 106.68) (width 0.25) (layer F.Cu) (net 15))
 (segment (start 114.808 110.998) (end 111.251999 107.441999) (width 0.25) (layer F.Cu) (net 15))
 (segment (start 114.808 127.762) (end 114.808 110.998) (width 0.25) (layer F.Cu) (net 15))
 (segment (start 110.49 132.08) (end 114.808 127.762) (width 0.25) (layer F.Cu) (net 15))
 (segment (start 113.538 145.880762) (end 113.538 135.128) (width 0.25) (layer F.Cu) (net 15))
 (segment (start 111.011761 148.407001) (end 113.538 145.880762) (width 0.25) (layer F.Cu) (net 15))
 (segment (start 110.334237 148.407001) (end 111.011761 148.407001) (width 0.25) (layer F.Cu) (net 15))
 (segment (start 53.522999 140.787001) (end 53.522999 149.534999) (width 0.25) (layer F.Cu) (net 15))
 (segment (start 54.61 139.7) (end 53.522999 140.787001) (width 0.25) (layer F.Cu) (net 15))
 (segment (start 108.627238 150.114) (end 110.334237 148.407001) (width 0.25) (layer F.Cu) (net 15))
 (segment (start 113.538 135.128) (end 110.49 132.08) (width 0.25) (layer F.Cu) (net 15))
 (segment (start 53.522999 149.534999) (end 54.102 150.114) (width 0.25) (layer F.Cu) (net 15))
 (segment (start 54.102 150.114) (end 108.627238 150.114) (width 0.25) (layer F.Cu) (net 15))
 (segment (start 55.371999 126.238001) (end 54.61 127) (width 0.25) (layer F.Cu) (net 11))
 (segment (start 60.865001 120.744999) (end 55.371999 126.238001) (width 0.25) (layer F.Cu) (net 11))
 (segment (start 106.585001 120.744999) (end 60.865001 120.744999) (width 0.25) (layer F.Cu) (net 11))
 (segment (start 110.49 116.84) (end 106.585001 120.744999) (width 0.25) (layer F.Cu) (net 11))
 (segment (start 111.251999 117.601999) (end 110.49 116.84) (width 0.25) (layer B.Cu) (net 11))
 (segment (start 114.046 132.672762) (end 114.046 120.396) (width 0.25) (layer B.Cu) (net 11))
 (segment (start 107.95 139.7) (end 107.95 138.091238) (width 0.25) (layer B.Cu) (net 11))
 (segment (start 107.95 138.091238) (end 110.334237 135.707001) (width 0.25) (layer B.Cu) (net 11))
 (segment (start 110.49 142.24) (end 107.95 139.7) (width 0.25) (layer B.Cu) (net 11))
 (segment (start 111.011761 135.707001) (end 114.046 132.672762) (width 0.25) (layer B.Cu) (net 11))
 (segment (start 114.046 120.396) (end 111.251999 117.601999) (width 0.25) (layer B.Cu) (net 11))
 (segment (start 110.334237 135.707001) (end 111.011761 135.707001) (width 0.25) (layer B.Cu) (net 11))
 (segment (start 53.522999 125.547001) (end 53.848001 125.221999) (width 0.25) (layer F.Cu) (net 10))
 (segment (start 53.522999 127.521761) (end 53.522999 125.547001) (width 0.25) (layer F.Cu) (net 10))
 (segment (start 54.088239 128.087001) (end 53.522999 127.521761) (width 0.25) (layer F.Cu) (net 10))
 (segment (start 55.131761 128.087001) (end 54.088239 128.087001) (width 0.25) (layer F.Cu) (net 10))
 (segment (start 59.933763 123.284999) (end 55.131761 128.087001) (width 0.25) (layer F.Cu) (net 10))
 (segment (start 53.848001 125.221999) (end 54.61 124.46) (width 0.25) (layer F.Cu) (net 10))
 (segment (start 86.924001 123.284999) (end 59.933763 123.284999) (width 0.25) (layer F.Cu) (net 10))
 (segment (start 88.739009 121.469991) (end 86.924001 123.284999) (width 0.25) (layer F.Cu) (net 10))
 (segment (start 108.400009 121.469991) (end 88.739009 121.469991) (width 0.25) (layer F.Cu) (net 10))
 (segment (start 110.49 119.38) (end 108.400009 121.469991) (width 0.25) (layer F.Cu) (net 10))
 (segment (start 107.499991 122.370009) (end 109.728001 120.141999) (width 0.25) (layer B.Cu) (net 10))
 (segment (start 107.499991 140.858753) (end 107.499991 122.370009) (width 0.25) (layer B.Cu) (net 10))
 (segment (start 109.728001 120.141999) (end 110.49 119.38) (width 0.25) (layer B.Cu) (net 10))
 (segment (start 110.49 143.848762) (end 107.499991 140.858753) (width 0.25) (layer B.Cu) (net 10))
 (segment (start 110.49 144.78) (end 110.49 143.848762) (width 0.25) (layer B.Cu) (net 10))
 (segment (start 123.19 121.92) (end 121.92 121.92) (width 0.25) (layer F.Cu) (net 7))
 (segment (start 121.902999 121.902999) (end 120.632999 121.902999) (width 0.25) (layer F.Cu) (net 7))
 (segment (start 121.92 121.92) (end 121.902999 121.902999) (width 0.25) (layer F.Cu) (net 7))
 (segment (start 120.632999 121.902999) (end 118.11 119.38) (width 0.25) (layer F.Cu) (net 7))
 (segment (start 118.11 119.38) (end 118.11 105.41) (width 0.25) (layer F.Cu) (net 7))
 (segment (start 118.11 105.41) (end 116.84 104.14) (width 0.25) (layer F.Cu) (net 7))
 (segment (start 67.31 104.14) (end 54.61 116.84) (width 0.25) (layer F.Cu) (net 7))
 (segment (start 116.84 104.14) (end 67.31 104.14) (width 0.25) (layer F.Cu) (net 7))
 (segment (start 123.19 147.32) (end 119.38 147.32) (width 0.25) (layer F.Cu) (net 20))
 (segment (start 119.38 147.32) (end 117.927001 148.772999) (width 0.25) (layer F.Cu) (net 20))
 (segment (start 107.611238 151.13) (end 57.010108 151.13) (width 0.25) (layer F.Cu) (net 20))
 (segment (start 57.010108 151.13) (end 53.34 151.13) (width 0.25) (layer F.Cu) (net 20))
 (segment (start 53.34 151.13) (end 52.07 149.86) (width 0.25) (layer F.Cu) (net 20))
 (segment (start 52.07 149.86) (end 52.07 116.64113) (width 0.25) (layer F.Cu) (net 20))
 (segment (start 52.07 116.64113) (end 52.07 115.57) (width 0.25) (layer F.Cu) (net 20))
 (segment (start 53.53237 114.10113) (end 52.07 115.5635) (width 0.25) (layer F.Cu) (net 20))
 (segment (start 54.61 114.10113) (end 53.53237 114.10113) (width 0.25) (layer F.Cu) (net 20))
 (segment (start 107.611238 151.13) (end 115.57 151.13) (width 0.25) (layer F.Cu) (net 20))
 (segment (start 115.57 151.13) (end 118.11 148.59) (width 0.25) (layer F.Cu) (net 20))
 (segment (start 80.771999 123.698001) (end 80.01 124.46) (width 0.25) (layer B.Cu) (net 22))
 (segment (start 81.185001 123.284999) (end 80.771999 123.698001) (width 0.25) (layer B.Cu) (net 22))
 (segment (start 88.740001 123.284999) (end 81.185001 123.284999) (width 0.25) (layer B.Cu) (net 22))
 (segment (start 109.402999 143.947997) (end 88.740001 123.284999) (width 0.25) (layer B.Cu) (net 22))
 (segment (start 109.402999 146.232999) (end 109.402999 143.947997) (width 0.25) (layer B.Cu) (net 22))
 (segment (start 110.49 147.32) (end 109.402999 146.232999) (width 0.25) (layer B.Cu) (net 22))
 (segment (start 80.771999 126.238001) (end 80.01 127) (width 0.25) (layer B.Cu) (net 21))
 (segment (start 100.235001 136.595999) (end 89.464001 125.824999) (width 0.25) (layer B.Cu) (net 21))
 (segment (start 89.464001 125.824999) (end 81.185001 125.824999) (width 0.25) (layer B.Cu) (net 21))
 (segment (start 100.235001 139.350003) (end 100.235001 136.595999) (width 0.25) (layer B.Cu) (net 21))
 (segment (start 101.759999 140.875001) (end 100.235001 139.350003) (width 0.25) (layer B.Cu) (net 21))
 (segment (start 103.244003 140.875001) (end 101.759999 140.875001) (width 0.25) (layer B.Cu) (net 21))
 (segment (start 104.045001 143.415001) (end 104.045001 141.675999) (width 0.25) (layer B.Cu) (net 21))
 (segment (start 81.185001 125.824999) (end 80.771999 126.238001) (width 0.25) (layer B.Cu) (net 21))
 (segment (start 104.045001 141.675999) (end 103.244003 140.875001) (width 0.25) (layer B.Cu) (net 21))
 (segment (start 110.49 149.86) (end 104.045001 143.415001) (width 0.25) (layer B.Cu) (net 21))
 (segment (start 102.87 121.92) (end 88.9 135.89) (width 0.25) (layer F.Cu) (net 9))
 (segment (start 110.49 121.92) (end 102.87 121.92) (width 0.25) (layer F.Cu) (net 9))
 (segment (start 83.82 135.89) (end 80.01 132.08) (width 0.25) (layer F.Cu) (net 9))
 (segment (start 88.9 135.89) (end 83.82 135.89) (width 0.25) (layer F.Cu) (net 9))
 (segment (start 110.49 124.46) (end 101.6 124.46) (width 0.25) (layer F.Cu) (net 8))
 (segment (start 101.6 124.46) (end 88.9 137.16) (width 0.25) (layer F.Cu) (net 8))
 (segment (start 88.9 137.16) (end 82.55 137.16) (width 0.25) (layer F.Cu) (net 8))
 (segment (start 82.55 137.16) (end 80.01 134.62) (width 0.25) (layer F.Cu) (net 8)))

